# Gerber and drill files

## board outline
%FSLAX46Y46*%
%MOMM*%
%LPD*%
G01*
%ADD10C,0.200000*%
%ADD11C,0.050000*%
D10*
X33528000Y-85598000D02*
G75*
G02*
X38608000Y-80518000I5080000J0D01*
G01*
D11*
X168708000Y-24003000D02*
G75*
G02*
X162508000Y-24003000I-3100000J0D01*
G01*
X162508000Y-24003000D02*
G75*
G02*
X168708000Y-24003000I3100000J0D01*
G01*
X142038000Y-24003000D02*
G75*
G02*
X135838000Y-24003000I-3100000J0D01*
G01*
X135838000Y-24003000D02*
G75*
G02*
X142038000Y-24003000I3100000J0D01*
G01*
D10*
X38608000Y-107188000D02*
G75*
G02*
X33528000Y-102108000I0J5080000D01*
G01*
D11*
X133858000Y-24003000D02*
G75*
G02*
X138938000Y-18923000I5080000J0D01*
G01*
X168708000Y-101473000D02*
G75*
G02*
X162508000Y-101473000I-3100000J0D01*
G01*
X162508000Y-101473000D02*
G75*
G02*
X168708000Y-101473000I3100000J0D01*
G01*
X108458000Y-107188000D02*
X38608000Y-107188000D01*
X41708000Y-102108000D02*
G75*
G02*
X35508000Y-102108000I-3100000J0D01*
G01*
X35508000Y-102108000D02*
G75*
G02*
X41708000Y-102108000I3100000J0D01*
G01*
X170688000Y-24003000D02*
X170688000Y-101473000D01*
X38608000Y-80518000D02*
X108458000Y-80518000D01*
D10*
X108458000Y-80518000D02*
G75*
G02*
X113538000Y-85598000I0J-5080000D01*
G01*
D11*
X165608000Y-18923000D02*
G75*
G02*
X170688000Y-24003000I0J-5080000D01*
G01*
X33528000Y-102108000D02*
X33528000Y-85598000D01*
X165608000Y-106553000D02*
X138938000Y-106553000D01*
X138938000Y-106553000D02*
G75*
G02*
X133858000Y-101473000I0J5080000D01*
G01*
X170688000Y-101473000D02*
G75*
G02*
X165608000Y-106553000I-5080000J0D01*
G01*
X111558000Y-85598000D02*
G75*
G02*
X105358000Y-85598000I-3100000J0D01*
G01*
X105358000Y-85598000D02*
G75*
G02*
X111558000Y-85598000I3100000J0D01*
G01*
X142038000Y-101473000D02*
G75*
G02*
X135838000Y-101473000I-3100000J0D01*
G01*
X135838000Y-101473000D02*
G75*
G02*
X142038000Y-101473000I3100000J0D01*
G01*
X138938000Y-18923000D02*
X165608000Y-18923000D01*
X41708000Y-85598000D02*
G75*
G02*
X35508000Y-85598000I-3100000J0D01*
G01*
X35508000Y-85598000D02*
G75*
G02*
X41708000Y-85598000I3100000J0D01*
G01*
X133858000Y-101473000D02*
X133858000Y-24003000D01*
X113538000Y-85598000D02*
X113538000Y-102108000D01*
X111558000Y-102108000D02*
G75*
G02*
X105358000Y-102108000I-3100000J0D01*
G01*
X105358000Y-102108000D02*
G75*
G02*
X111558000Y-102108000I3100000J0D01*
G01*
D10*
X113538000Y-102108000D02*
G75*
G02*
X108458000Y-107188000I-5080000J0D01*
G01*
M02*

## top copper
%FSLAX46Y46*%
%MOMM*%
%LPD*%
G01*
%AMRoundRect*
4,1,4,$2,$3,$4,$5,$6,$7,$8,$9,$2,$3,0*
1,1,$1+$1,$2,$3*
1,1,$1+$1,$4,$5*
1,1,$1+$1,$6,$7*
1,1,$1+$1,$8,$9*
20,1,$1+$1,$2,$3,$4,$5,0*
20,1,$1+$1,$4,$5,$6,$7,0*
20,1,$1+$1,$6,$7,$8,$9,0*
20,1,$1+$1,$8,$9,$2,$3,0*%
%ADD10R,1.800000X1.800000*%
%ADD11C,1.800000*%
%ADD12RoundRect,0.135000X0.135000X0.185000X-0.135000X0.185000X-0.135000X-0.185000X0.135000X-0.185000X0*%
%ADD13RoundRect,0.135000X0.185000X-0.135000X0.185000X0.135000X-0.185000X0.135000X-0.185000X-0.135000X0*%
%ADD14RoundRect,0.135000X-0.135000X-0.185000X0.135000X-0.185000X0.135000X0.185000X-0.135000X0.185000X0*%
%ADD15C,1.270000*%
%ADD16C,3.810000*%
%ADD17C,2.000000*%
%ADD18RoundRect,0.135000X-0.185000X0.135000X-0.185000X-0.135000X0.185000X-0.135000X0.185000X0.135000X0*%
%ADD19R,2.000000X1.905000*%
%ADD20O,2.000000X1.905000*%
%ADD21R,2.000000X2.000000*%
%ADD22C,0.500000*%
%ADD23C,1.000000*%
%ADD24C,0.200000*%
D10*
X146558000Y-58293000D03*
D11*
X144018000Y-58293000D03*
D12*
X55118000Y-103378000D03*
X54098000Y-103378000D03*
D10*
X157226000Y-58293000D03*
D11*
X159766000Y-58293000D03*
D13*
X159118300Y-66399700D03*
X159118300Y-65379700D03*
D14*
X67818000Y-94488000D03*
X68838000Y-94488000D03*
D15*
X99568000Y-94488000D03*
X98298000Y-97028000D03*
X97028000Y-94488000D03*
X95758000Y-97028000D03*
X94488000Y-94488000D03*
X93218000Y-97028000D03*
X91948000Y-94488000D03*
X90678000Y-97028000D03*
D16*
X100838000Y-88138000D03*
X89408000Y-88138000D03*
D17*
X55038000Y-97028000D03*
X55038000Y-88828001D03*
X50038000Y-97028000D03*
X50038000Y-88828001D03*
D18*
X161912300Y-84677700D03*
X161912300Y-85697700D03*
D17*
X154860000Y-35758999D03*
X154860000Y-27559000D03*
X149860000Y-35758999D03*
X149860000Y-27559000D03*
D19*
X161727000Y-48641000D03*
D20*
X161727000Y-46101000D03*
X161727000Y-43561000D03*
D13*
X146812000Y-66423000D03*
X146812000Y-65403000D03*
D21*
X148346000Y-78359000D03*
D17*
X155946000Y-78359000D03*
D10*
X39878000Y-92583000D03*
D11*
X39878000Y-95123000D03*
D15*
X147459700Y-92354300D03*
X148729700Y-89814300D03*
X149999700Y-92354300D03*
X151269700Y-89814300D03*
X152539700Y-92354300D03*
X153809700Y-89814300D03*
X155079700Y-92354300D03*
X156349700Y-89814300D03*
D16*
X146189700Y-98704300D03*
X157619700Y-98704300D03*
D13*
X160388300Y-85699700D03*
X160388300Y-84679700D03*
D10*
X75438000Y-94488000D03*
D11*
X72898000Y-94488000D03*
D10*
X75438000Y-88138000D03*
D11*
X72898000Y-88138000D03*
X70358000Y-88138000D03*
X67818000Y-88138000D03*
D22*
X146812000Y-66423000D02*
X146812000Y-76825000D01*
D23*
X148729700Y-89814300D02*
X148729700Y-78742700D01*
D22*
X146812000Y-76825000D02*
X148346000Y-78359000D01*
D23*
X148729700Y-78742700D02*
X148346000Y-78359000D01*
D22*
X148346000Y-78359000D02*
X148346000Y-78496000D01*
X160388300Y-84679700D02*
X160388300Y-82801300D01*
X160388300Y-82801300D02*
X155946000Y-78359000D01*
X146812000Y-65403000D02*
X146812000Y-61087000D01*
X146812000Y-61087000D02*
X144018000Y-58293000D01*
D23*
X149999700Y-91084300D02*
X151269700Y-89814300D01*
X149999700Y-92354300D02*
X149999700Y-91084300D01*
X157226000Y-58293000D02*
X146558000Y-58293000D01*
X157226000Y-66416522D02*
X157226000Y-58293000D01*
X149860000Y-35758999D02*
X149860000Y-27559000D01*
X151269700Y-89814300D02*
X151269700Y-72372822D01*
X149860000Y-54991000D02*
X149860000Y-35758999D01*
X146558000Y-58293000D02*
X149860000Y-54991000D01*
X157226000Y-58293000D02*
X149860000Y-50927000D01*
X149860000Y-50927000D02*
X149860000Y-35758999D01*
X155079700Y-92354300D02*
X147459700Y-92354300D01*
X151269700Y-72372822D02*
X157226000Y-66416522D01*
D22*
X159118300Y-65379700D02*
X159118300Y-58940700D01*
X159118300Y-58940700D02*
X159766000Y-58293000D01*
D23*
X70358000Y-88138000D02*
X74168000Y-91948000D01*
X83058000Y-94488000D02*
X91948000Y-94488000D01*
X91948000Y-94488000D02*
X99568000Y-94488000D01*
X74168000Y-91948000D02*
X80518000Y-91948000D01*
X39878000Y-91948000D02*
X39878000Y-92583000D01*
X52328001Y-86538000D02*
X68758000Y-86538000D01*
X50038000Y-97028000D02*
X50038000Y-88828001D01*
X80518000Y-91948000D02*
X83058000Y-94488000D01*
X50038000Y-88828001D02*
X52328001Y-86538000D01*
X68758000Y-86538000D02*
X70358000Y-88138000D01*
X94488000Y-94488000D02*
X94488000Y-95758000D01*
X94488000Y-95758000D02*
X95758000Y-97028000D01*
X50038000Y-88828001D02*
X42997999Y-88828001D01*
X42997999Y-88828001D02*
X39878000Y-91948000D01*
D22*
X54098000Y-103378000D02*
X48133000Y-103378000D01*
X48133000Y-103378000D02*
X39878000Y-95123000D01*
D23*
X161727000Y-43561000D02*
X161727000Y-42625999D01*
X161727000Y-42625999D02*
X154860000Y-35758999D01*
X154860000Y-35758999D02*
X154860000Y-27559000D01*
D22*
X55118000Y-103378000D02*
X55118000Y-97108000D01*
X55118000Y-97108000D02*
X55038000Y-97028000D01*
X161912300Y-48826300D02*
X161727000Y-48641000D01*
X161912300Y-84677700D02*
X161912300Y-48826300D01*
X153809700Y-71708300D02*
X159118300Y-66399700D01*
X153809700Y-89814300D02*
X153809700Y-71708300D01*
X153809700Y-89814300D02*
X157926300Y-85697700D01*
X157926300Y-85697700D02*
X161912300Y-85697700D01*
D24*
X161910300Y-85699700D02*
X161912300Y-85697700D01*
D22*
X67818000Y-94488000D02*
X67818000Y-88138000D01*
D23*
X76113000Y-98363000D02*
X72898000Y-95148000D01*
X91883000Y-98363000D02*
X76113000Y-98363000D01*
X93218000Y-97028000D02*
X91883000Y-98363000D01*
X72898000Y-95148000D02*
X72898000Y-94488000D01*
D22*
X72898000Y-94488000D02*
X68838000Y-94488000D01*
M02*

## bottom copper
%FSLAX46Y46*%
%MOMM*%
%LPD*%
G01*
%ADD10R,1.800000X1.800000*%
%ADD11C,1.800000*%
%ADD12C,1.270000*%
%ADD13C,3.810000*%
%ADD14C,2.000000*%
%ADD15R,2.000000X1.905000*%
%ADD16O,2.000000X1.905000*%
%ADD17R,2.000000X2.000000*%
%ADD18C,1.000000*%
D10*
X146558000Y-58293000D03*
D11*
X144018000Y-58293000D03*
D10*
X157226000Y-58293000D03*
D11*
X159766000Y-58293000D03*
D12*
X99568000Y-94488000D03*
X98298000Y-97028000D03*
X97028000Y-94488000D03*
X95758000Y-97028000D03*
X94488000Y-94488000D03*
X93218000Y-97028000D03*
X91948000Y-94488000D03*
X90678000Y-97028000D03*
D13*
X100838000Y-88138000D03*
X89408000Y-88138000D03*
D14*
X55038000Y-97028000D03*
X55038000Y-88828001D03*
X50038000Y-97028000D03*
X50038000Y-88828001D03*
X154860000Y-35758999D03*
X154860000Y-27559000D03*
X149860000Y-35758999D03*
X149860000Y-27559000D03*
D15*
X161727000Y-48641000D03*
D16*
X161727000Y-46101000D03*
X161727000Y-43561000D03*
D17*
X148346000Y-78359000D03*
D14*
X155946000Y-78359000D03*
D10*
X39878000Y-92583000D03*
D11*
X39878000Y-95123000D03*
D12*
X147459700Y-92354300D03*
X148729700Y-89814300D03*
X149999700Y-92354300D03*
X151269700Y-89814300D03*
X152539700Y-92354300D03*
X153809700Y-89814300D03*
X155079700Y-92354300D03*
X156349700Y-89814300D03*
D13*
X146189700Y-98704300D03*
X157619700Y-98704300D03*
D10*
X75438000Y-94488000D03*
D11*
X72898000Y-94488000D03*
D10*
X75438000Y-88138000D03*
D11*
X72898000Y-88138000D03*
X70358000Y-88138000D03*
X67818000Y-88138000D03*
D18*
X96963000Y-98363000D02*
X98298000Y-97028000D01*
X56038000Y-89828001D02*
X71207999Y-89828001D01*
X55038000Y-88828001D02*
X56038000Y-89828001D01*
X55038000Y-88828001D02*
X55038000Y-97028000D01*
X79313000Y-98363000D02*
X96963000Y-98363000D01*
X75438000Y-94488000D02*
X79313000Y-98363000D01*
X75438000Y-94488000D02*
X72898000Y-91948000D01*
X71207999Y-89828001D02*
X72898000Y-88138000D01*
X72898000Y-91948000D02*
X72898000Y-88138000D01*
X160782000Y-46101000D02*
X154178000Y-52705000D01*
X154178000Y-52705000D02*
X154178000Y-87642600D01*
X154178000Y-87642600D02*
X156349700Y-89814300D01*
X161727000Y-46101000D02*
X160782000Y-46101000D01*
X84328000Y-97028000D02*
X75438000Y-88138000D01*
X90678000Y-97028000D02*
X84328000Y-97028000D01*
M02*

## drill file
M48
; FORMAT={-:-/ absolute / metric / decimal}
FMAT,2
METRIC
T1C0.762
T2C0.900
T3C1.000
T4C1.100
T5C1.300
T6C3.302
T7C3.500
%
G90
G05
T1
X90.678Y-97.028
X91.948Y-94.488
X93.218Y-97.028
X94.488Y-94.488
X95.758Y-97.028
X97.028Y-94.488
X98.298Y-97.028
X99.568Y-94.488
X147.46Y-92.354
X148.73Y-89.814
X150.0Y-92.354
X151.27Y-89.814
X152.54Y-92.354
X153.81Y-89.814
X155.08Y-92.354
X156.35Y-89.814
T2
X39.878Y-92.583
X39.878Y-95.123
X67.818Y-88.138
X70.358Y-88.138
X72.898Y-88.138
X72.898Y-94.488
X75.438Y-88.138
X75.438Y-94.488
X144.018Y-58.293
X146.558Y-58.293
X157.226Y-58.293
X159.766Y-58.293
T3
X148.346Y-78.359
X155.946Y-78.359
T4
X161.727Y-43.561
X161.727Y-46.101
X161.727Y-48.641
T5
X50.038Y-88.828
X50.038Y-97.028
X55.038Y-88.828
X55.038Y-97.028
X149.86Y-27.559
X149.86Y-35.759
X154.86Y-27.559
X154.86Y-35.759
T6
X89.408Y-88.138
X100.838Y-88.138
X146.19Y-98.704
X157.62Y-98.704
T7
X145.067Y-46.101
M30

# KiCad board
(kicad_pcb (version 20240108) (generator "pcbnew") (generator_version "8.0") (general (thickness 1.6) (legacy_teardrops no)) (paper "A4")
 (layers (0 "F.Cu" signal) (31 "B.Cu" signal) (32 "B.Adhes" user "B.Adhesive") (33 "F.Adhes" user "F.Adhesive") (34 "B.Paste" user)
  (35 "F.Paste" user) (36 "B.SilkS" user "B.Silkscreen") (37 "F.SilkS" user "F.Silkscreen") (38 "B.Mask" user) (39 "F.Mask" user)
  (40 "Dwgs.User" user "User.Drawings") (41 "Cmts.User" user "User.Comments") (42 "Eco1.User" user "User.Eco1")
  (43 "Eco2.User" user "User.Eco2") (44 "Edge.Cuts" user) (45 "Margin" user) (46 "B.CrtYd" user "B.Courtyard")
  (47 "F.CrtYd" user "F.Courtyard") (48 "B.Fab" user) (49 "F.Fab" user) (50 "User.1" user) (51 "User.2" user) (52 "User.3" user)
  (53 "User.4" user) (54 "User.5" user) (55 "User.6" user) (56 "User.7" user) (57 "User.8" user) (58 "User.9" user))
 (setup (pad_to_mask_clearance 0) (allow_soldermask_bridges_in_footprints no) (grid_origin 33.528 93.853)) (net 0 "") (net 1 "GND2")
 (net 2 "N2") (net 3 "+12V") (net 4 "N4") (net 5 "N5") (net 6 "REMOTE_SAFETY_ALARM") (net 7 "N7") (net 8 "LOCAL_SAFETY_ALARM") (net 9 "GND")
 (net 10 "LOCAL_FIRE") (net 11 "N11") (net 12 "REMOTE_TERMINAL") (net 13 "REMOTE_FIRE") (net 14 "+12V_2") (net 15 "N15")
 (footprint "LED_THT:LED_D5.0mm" (layer "F.Cu") (at 146.558 58.293 180)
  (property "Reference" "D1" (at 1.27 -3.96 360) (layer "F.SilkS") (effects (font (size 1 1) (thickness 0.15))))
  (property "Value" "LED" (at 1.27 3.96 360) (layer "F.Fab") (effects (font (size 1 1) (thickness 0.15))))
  (pad "1" thru_hole rect (at 0 0 180) (size 1.8 1.8) (drill 0.9) (layers "*.Cu" "*.Mask") (remove_unused_layers no) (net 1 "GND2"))
  (pad "2" thru_hole circle (at 2.54 0 180) (size 1.8 1.8) (drill 0.9) (layers "*.Cu" "*.Mask") (remove_unused_layers no) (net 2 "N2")))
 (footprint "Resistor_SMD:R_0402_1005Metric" (layer "F.Cu") (at 54.608 103.378 180)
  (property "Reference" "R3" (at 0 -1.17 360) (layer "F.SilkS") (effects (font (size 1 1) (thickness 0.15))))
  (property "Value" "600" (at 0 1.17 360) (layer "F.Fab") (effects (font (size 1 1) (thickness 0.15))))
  (pad "1" smd roundrect (at -0.51 0 180) (size 0.54 0.64) (layers "F.Cu" "F.Paste" "F.Mask") (roundrect_rratio 0.25) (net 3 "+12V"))
  (pad "2" smd roundrect (at 0.51 0 180) (size 0.54 0.64) (layers "F.Cu" "F.Paste" "F.Mask") (roundrect_rratio 0.25) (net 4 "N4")))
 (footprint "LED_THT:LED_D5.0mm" (layer "F.Cu") (at 157.226 58.293)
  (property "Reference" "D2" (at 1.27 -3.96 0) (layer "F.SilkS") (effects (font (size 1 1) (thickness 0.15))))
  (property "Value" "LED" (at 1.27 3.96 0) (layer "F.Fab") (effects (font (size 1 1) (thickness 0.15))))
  (pad "1" thru_hole rect (at 0 0) (size 1.8 1.8) (drill 0.9) (layers "*.Cu" "*.Mask") (remove_unused_layers no) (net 1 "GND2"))
  (pad "2" thru_hole circle (at 2.54 0) (size 1.8 1.8) (drill 0.9) (layers "*.Cu" "*.Mask") (remove_unused_layers no) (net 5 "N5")))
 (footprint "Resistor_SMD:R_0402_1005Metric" (layer "F.Cu") (at 159.1183 65.8897 90)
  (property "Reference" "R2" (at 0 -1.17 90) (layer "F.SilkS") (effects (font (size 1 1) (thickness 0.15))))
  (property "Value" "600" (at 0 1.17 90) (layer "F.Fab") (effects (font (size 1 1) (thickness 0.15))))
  (pad "1" smd roundrect (at -0.51 0 90) (size 0.54 0.64) (layers "F.Cu" "F.Paste" "F.Mask") (roundrect_rratio 0.25)
   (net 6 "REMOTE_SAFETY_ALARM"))
  (pad "2" smd roundrect (at 0.51 0 90) (size 0.54 0.64) (layers "F.Cu" "F.Paste" "F.Mask") (roundrect_rratio 0.25) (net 5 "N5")))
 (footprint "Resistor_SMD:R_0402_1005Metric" (layer "F.Cu") (at 68.328 94.488)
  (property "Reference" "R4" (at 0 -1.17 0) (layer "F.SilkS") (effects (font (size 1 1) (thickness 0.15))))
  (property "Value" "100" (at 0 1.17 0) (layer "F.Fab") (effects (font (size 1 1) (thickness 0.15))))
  (pad "1" smd roundrect (at -0.51 0) (size 0.54 0.64) (layers "F.Cu" "F.Paste" "F.Mask") (roundrect_rratio 0.25) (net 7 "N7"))
  (pad "2" smd roundrect (at 0.51 0) (size 0.54 0.64) (layers "F.Cu" "F.Paste" "F.Mask") (roundrect_rratio 0.25)
   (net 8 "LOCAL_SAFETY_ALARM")))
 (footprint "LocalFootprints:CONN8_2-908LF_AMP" (layer "F.Cu") (at 99.568 94.488 180)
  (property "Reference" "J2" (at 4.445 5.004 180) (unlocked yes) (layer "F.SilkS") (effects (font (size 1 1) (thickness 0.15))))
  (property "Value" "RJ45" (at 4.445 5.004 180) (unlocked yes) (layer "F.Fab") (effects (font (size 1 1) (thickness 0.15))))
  (pad "1" thru_hole circle (at 0 0 180) (size 1.27 1.27) (drill 0.762) (layers "*.Cu" "*.Mask") (remove_unused_layers no) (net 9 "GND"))
  (pad "2" thru_hole circle (at 1.27 -2.54 180) (size 1.27 1.27) (drill 0.762) (layers "*.Cu" "*.Mask") (remove_unused_layers no)
   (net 3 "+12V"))
  (pad "3" thru_hole circle (at 2.54 0 180) (size 1.27 1.27) (drill 0.762) (layers "*.Cu" "*.Mask") (remove_unused_layers no) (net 9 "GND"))
  (pad "4" thru_hole circle (at 3.81 -2.54 180) (size 1.27 1.27) (drill 0.762) (layers "*.Cu" "*.Mask") (remove_unused_layers no)
   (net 9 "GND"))
  (pad "5" thru_hole circle (at 5.08 0 180) (size 1.27 1.27) (drill 0.762) (layers "*.Cu" "*.Mask") (remove_unused_layers no) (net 9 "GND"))
  (pad "6" thru_hole circle (at 6.35 -2.54 180) (size 1.27 1.27) (drill 0.762) (layers "*.Cu" "*.Mask") (remove_unused_layers no)
   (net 8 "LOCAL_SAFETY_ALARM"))
  (pad "7" thru_hole circle (at 7.62 0 180) (size 1.27 1.27) (drill 0.762) (layers "*.Cu" "*.Mask") (remove_unused_layers no) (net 9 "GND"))
  (pad "8" thru_hole circle (at 8.89 -2.54 180) (size 1.27 1.27) (drill 0.762) (layers "*.Cu" "*.Mask") (remove_unused_layers no)
   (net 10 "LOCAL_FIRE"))
  (pad "9" thru_hole circle (at -1.27 6.35 270) (size 3.81 3.81) (drill 3.302) (layers "*.Cu" "*.Mask") (remove_unused_layers no))
  (pad "10" thru_hole circle (at 10.16 6.35 270) (size 3.81 3.81) (drill 3.302) (layers "*.Cu" "*.Mask") (remove_unused_layers no)))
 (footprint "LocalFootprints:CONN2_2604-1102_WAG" (layer "F.Cu") (at 55.038 97.028 180)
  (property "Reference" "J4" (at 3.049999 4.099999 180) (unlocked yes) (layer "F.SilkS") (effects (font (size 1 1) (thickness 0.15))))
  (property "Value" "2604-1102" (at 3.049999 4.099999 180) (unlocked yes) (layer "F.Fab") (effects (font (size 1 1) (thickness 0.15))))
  (pad "1" thru_hole circle (at 0 0 180) (size 2 2) (drill 1.3) (layers "*.Cu" "*.Mask") (remove_unused_layers no) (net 3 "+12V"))
  (pad "2" thru_hole circle (at 0 8.199999 180) (size 2 2) (drill 1.3) (layers "*.Cu" "*.Mask") (remove_unused_layers no) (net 3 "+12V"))
  (pad "3" thru_hole circle (at 5 0 180) (size 2 2) (drill 1.3) (layers "*.Cu" "*.Mask") (remove_unused_layers no) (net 9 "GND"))
  (pad "4" thru_hole circle (at 5 8.199999 180) (size 2 2) (drill 1.3) (layers "*.Cu" "*.Mask") (remove_unused_layers no) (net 9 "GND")))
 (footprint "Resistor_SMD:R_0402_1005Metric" (layer "F.Cu") (at 161.9123 85.1877 -90)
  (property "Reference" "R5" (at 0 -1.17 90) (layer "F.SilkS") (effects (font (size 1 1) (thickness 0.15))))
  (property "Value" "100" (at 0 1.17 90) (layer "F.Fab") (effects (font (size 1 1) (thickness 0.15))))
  (pad "1" smd roundrect (at -0.51 0 270) (size 0.54 0.64) (layers "F.Cu" "F.Paste" "F.Mask") (roundrect_rratio 0.25) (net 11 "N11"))
  (pad "2" smd roundrect (at 0.51 0 270) (size 0.54 0.64) (layers "F.Cu" "F.Paste" "F.Mask") (roundrect_rratio 0.25)
   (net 6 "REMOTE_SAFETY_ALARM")))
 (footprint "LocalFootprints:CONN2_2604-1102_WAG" (layer "F.Cu") (at 154.86 35.758999 180)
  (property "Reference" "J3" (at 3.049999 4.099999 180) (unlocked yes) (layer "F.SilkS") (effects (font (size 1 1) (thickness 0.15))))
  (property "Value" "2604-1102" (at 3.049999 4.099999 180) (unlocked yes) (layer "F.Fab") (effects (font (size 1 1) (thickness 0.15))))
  (pad "1" thru_hole circle (at 0 0 180) (size 2 2) (drill 1.3) (layers "*.Cu" "*.Mask") (remove_unused_layers no)
   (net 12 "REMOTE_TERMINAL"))
  (pad "2" thru_hole circle (at 0 8.199999 180) (size 2 2) (drill 1.3) (layers "*.Cu" "*.Mask") (remove_unused_layers no)
   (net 12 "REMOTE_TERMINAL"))
  (pad "3" thru_hole circle (at 5 0 180) (size 2 2) (drill 1.3) (layers "*.Cu" "*.Mask") (remove_unused_layers no) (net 1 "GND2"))
  (pad "4" thru_hole circle (at 5 8.199999 180) (size 2 2) (drill 1.3) (layers "*.Cu" "*.Mask") (remove_unused_layers no) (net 1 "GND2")))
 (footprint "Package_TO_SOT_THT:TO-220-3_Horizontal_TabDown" (layer "F.Cu") (at 161.727 48.641 90)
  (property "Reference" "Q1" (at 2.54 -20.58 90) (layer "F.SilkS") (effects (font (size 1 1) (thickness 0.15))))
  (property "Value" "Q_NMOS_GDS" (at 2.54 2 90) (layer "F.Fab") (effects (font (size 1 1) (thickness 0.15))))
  (pad "" np_thru_hole oval (at 2.54 -16.66 90) (size 3.5 3.5) (drill 3.5) (layers "*.Cu" "*.Mask"))
  (pad "1" thru_hole rect (at 0 0 90) (size 1.905 2) (drill 1.1) (layers "*.Cu" "*.Mask") (remove_unused_layers no) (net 11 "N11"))
  (pad "2" thru_hole oval (at 2.54 0 90) (size 1.905 2) (drill 1.1) (layers "*.Cu" "*.Mask") (remove_unused_layers no)
   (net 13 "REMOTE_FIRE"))
  (pad "3" thru_hole oval (at 5.08 0 90) (size 1.905 2) (drill 1.1) (layers "*.Cu" "*.Mask") (remove_unused_layers no)
   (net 12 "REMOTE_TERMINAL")))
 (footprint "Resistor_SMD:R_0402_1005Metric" (layer "F.Cu") (at 146.812 65.913 90)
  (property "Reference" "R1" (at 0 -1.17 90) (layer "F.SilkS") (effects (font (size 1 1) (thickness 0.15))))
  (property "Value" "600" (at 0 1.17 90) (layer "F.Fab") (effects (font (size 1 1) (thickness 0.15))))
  (pad "1" smd roundrect (at -0.51 0 90) (size 0.54 0.64) (layers "F.Cu" "F.Paste" "F.Mask") (roundrect_rratio 0.25) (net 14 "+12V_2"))
  (pad "2" smd roundrect (at 0.51 0 90) (size 0.54 0.64) (layers "F.Cu" "F.Paste" "F.Mask") (roundrect_rratio 0.25) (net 2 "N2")))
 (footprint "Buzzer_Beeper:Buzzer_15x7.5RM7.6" (layer "F.Cu") (at 148.346 78.359)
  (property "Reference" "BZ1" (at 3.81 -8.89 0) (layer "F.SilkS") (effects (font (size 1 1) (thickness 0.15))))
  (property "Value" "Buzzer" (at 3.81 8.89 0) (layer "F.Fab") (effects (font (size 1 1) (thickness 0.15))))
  (pad "1" thru_hole rect (at 0 0) (size 2 2) (drill 1) (layers "*.Cu" "*.Mask") (remove_unused_layers no) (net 14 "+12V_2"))
  (pad "2" thru_hole circle (at 7.6 0) (size 2 2) (drill 1) (layers "*.Cu" "*.Mask") (remove_unused_layers no) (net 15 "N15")))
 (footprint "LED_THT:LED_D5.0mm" (layer "F.Cu") (at 39.878 92.583 -90)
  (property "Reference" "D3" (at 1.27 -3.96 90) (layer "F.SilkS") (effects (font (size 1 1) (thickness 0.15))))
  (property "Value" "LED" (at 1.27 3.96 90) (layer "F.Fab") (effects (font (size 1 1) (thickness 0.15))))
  (pad "1" thru_hole rect (at 0 0 270) (size 1.8 1.8) (drill 0.9) (layers "*.Cu" "*.Mask") (remove_unused_layers no) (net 9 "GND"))
  (pad "2" thru_hole circle (at 2.54 0 270) (size 1.8 1.8) (drill 0.9) (layers "*.Cu" "*.Mask") (remove_unused_layers no) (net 4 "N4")))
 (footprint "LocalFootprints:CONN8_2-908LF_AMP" (layer "F.Cu") (at 147.4597 92.3543)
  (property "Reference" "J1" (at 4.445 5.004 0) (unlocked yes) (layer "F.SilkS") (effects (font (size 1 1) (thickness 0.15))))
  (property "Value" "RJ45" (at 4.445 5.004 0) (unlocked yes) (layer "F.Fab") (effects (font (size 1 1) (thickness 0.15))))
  (pad "1" thru_hole circle (at 0 0) (size 1.27 1.27) (drill 0.762) (layers "*.Cu" "*.Mask") (remove_unused_layers no) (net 1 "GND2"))
  (pad "2" thru_hole circle (at 1.27 -2.54) (size 1.27 1.27) (drill 0.762) (layers "*.Cu" "*.Mask") (remove_unused_layers no)
   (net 14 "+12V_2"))
  (pad "3" thru_hole circle (at 2.54 0) (size 1.27 1.27) (drill 0.762) (layers "*.Cu" "*.Mask") (remove_unused_layers no) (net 1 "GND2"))
  (pad "4" thru_hole circle (at 3.81 -2.54) (size 1.27 1.27) (drill 0.762) (layers "*.Cu" "*.Mask") (remove_unused_layers no) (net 1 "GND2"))
  (pad "5" thru_hole circle (at 5.08 0) (size 1.27 1.27) (drill 0.762) (layers "*.Cu" "*.Mask") (remove_unused_layers no) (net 1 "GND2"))
  (pad "6" thru_hole circle (at 6.35 -2.54) (size 1.27 1.27) (drill 0.762) (layers "*.Cu" "*.Mask") (remove_unused_layers no)
   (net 6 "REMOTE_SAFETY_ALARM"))
  (pad "7" thru_hole circle (at 7.62 0) (size 1.27 1.27) (drill 0.762) (layers "*.Cu" "*.Mask") (remove_unused_layers no) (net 1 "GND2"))
  (pad "8" thru_hole circle (at 8.89 -2.54) (size 1.27 1.27) (drill 0.762) (layers "*.Cu" "*.Mask") (remove_unused_layers no)
   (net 13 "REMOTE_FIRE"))
  (pad "9" thru_hole circle (at -1.27 6.35 90) (size 3.81 3.81) (drill 3.302) (layers "*.Cu" "*.Mask") (remove_unused_layers no))
  (pad "10" thru_hole circle (at 10.16 6.35 90) (size 3.81 3.81) (drill 3.302) (layers "*.Cu" "*.Mask") (remove_unused_layers no)))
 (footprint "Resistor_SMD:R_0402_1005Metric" (layer "F.Cu") (at 160.3883 85.1897 90)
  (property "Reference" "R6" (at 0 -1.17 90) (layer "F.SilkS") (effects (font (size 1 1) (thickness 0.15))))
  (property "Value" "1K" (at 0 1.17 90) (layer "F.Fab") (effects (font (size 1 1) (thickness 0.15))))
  (pad "1" smd roundrect (at -0.51 0 90) (size 0.54 0.64) (layers "F.Cu" "F.Paste" "F.Mask") (roundrect_rratio 0.25)
   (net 6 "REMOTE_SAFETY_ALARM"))
  (pad "2" smd roundrect (at 0.51 0 90) (size 0.54 0.64) (layers "F.Cu" "F.Paste" "F.Mask") (roundrect_rratio 0.25) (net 15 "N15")))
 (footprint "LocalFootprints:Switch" (layer "B.Cu") (at 75.438 94.488 180)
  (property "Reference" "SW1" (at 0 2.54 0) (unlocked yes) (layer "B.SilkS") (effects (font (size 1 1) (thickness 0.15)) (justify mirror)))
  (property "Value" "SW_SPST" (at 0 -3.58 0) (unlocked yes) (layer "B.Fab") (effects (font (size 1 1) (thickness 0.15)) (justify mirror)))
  (pad "1" thru_hole rect (at 0 0 180) (size 1.8 1.8) (drill 0.9) (layers "*.Cu" "*.Mask") (remove_unused_layers no) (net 3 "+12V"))
  (pad "2" thru_hole circle (at 2.54 0 180) (size 1.8 1.8) (drill 0.9) (layers "*.Cu" "*.Mask") (remove_unused_layers no)
   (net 8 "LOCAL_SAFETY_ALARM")))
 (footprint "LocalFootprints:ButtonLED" (layer "B.Cu") (at 75.438 88.138 180)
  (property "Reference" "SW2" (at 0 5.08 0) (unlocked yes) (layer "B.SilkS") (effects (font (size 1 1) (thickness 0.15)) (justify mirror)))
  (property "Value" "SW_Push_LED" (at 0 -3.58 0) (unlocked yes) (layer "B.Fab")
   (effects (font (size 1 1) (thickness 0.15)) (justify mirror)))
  (pad "1" thru_hole rect (at 0 0 180) (size 1.8 1.8) (drill 0.9) (layers "*.Cu" "*.Mask") (remove_unused_layers no) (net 10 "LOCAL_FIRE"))
  (pad "2" thru_hole circle (at 2.54 0 180) (size 1.8 1.8) (drill 0.9) (layers "*.Cu" "*.Mask") (remove_unused_layers no) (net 3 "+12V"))
  (pad "3" thru_hole circle (at 5.08 0 180) (size 1.8 1.8) (drill 0.9) (layers "*.Cu" "*.Mask") (remove_unused_layers no) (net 9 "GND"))
  (pad "4" thru_hole circle (at 7.62 0 180) (size 1.8 1.8) (drill 0.9) (layers "*.Cu" "*.Mask") (remove_unused_layers no) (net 7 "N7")))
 (gr_arc (start 33.528 85.598) (mid 35.015898 82.005898) (end 38.608 80.518) (stroke (width 0.2) (type default)) (layer "Edge.Cuts"))
 (gr_circle (center 165.608 24.003) (end 168.708 24.003) (stroke (width 0.05) (type default)) (fill none) (layer "Edge.Cuts"))
 (gr_circle (center 138.938 24.003) (end 142.038 24.003) (stroke (width 0.05) (type default)) (fill none) (layer "Edge.Cuts"))
 (gr_arc (start 38.608 107.188) (mid 35.015898 105.700102) (end 33.528 102.108) (stroke (width 0.2) (type default)) (layer "Edge.Cuts"))
 (gr_arc (start 133.858 24.003) (mid 135.345898 20.410898) (end 138.938 18.923) (stroke (width 0.05) (type default)) (layer "Edge.Cuts"))
 (gr_circle (center 165.608 101.473) (end 168.708 101.473) (stroke (width 0.05) (type default)) (fill none) (layer "Edge.Cuts"))
 (gr_line (start 108.458 107.188) (end 38.608 107.188) (stroke (width 0.05) (type default)) (layer "Edge.Cuts"))
 (gr_circle (center 38.608 102.108) (end 41.708 102.108) (stroke (width 0.05) (type default)) (fill none) (layer "Edge.Cuts"))
 (gr_line (start 170.688 24.003) (end 170.688 101.473) (stroke (width 0.05) (type default)) (layer "Edge.Cuts"))
 (gr_line (start 38.608 80.518) (end 108.458 80.518) (stroke (width 0.05) (type default)) (layer "Edge.Cuts"))
 (gr_arc (start 108.458 80.518) (mid 112.050102 82.005898) (end 113.538 85.598) (stroke (width 0.2) (type default)) (layer "Edge.Cuts"))
 (gr_arc (start 165.608 18.923) (mid 169.200102 20.410898) (end 170.688 24.003) (stroke (width 0.05) (type default)) (layer "Edge.Cuts"))
 (gr_line (start 33.528 102.108) (end 33.528 85.598) (stroke (width 0.05) (type default)) (layer "Edge.Cuts"))
 (gr_line (start 165.608 106.553) (end 138.938 106.553) (stroke (width 0.05) (type default)) (layer "Edge.Cuts"))
 (gr_arc (start 138.938 106.553) (mid 135.345898 105.065102) (end 133.858 101.473) (stroke (width 0.05) (type default)) (layer "Edge.Cuts"))
 (gr_arc (start 170.688 101.473) (mid 169.200102 105.065102) (end 165.608 106.553) (stroke (width 0.05) (type default)) (layer "Edge.Cuts"))
 (gr_circle (center 108.458 85.598) (end 111.558 85.598) (stroke (width 0.05) (type default)) (fill none) (layer "Edge.Cuts"))
 (gr_circle (center 138.938 101.473) (end 142.038 101.473) (stroke (width 0.05) (type default)) (fill none) (layer "Edge.Cuts"))
 (gr_line (start 138.938 18.923) (end 165.608 18.923) (stroke (width 0.05) (type default)) (layer "Edge.Cuts"))
 (gr_circle (center 38.608 85.598) (end 41.708 85.598) (stroke (width 0.05) (type default)) (fill none) (layer "Edge.Cuts"))
 (gr_line (start 133.858 101.473) (end 133.858 24.003) (stroke (width 0.05) (type default)) (layer "Edge.Cuts"))
 (gr_line (start 113.538 85.598) (end 113.538 102.108) (stroke (width 0.05) (type default)) (layer "Edge.Cuts"))
 (gr_circle (center 108.458 102.108) (end 111.558 102.108) (stroke (width 0.05) (type default)) (fill none) (layer "Edge.Cuts"))
 (gr_arc (start 113.538 102.108) (mid 112.050102 105.700102) (end 108.458 107.188) (stroke (width 0.2) (type default)) (layer "Edge.Cuts"))
 (segment (start 146.812 66.423) (end 146.812 76.825) (width 0.5) (layer "F.Cu") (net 14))
 (segment (start 148.7297 89.8143) (end 148.7297 78.7427) (width 1) (layer "F.Cu") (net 14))
 (segment (start 146.812 76.825) (end 148.346 78.359) (width 0.5) (layer "F.Cu") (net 14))
 (segment (start 148.7297 78.7427) (end 148.346 78.359) (width 1) (layer "F.Cu") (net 14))
 (segment (start 148.346 78.359) (end 148.346 78.496) (width 0.5) (layer "F.Cu") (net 14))
 (segment (start 160.3883 84.6797) (end 160.3883 82.8013) (width 0.5) (layer "F.Cu") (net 15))
 (segment (start 160.3883 82.8013) (end 155.946 78.359) (width 0.5) (layer "F.Cu") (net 15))
 (segment (start 146.812 65.403) (end 146.812 61.087) (width 0.5) (layer "F.Cu") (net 2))
 (segment (start 146.812 61.087) (end 144.018 58.293) (width 0.5) (layer "F.Cu") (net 2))
 (segment (start 149.9997 91.0843) (end 151.2697 89.8143) (width 1) (layer "F.Cu") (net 1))
 (segment (start 149.9997 92.3543) (end 149.9997 91.0843) (width 1) (layer "F.Cu") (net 1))
 (segment (start 157.226 58.293) (end 146.558 58.293) (width 1) (layer "F.Cu") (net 1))
 (segment (start 157.226 66.416522) (end 157.226 58.293) (width 1) (layer "F.Cu") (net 1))
 (segment (start 149.86 35.758999) (end 149.86 27.559) (width 1) (layer "F.Cu") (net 1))
 (segment (start 151.2697 89.8143) (end 151.2697 72.372822) (width 1) (layer "F.Cu") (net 1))
 (segment (start 149.86 54.991) (end 149.86 35.758999) (width 1) (layer "F.Cu") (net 1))
 (segment (start 146.558 58.293) (end 149.86 54.991) (width 1) (layer "F.Cu") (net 1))
 (segment (start 157.226 58.293) (end 149.86 50.927) (width 1) (layer "F.Cu") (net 1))
 (segment (start 149.86 50.927) (end 149.86 35.758999) (width 1) (layer "F.Cu") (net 1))
 (segment (start 155.0797 92.3543) (end 147.4597 92.3543) (width 1) (layer "F.Cu") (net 1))
 (segment (start 151.2697 72.372822) (end 157.226 66.416522) (width 1) (layer "F.Cu") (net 1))
 (segment (start 159.1183 65.3797) (end 159.1183 58.9407) (width 0.5) (layer "F.Cu") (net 5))
 (segment (start 159.1183 58.9407) (end 159.766 58.293) (width 0.5) (layer "F.Cu") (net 5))
 (segment (start 70.358 88.138) (end 74.168 91.948) (width 1) (layer "F.Cu") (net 9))
 (segment (start 83.058 94.488) (end 91.948 94.488) (width 1) (layer "F.Cu") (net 9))
 (segment (start 91.948 94.488) (end 99.568 94.488) (width 1) (layer "F.Cu") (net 9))
 (segment (start 74.168 91.948) (end 80.518 91.948) (width 1) (layer "F.Cu") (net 9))
 (segment (start 39.878 91.948) (end 39.878 92.583) (width 1) (layer "F.Cu") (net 9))
 (segment (start 52.328001 86.538) (end 68.758 86.538) (width 1) (layer "F.Cu") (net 9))
 (segment (start 50.038 97.028) (end 50.038 88.828001) (width 1) (layer "F.Cu") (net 9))
 (segment (start 80.518 91.948) (end 83.058 94.488) (width 1) (layer "F.Cu") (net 9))
 (segment (start 50.038 88.828001) (end 52.328001 86.538) (width 1) (layer "F.Cu") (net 9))
 (segment (start 68.758 86.538) (end 70.358 88.138) (width 1) (layer "F.Cu") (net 9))
 (segment (start 94.488 94.488) (end 94.488 95.758) (width 1) (layer "F.Cu") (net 9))
 (segment (start 94.488 95.758) (end 95.758 97.028) (width 1) (layer "F.Cu") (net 9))
 (segment (start 50.038 88.828001) (end 42.997999 88.828001) (width 1) (layer "F.Cu") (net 9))
 (segment (start 42.997999 88.828001) (end 39.878 91.948) (width 1) (layer "F.Cu") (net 9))
 (segment (start 54.098 103.378) (end 48.133 103.378) (width 0.5) (layer "F.Cu") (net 4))
 (segment (start 48.133 103.378) (end 39.878 95.123) (width 0.5) (layer "F.Cu") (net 4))
 (segment (start 161.727 43.561) (end 161.727 42.625999) (width 1) (layer "F.Cu") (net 12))
 (segment (start 161.727 42.625999) (end 154.86 35.758999) (width 1) (layer "F.Cu") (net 12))
 (segment (start 154.86 35.758999) (end 154.86 27.559) (width 1) (layer "F.Cu") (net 12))
 (segment (start 55.118 103.378) (end 55.118 97.108) (width 0.5) (layer "F.Cu") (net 3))
 (segment (start 55.118 97.108) (end 55.038 97.028) (width 0.5) (layer "F.Cu") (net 3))
 (segment (start 96.963 98.363) (end 98.298 97.028) (width 1) (layer "B.Cu") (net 3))
 (segment (start 56.038 89.828001) (end 71.207999 89.828001) (width 1) (layer "B.Cu") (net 3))
 (segment (start 55.038 88.828001) (end 56.038 89.828001) (width 1) (layer "B.Cu") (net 3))
 (segment (start 55.038 88.828001) (end 55.038 97.028) (width 1) (layer "B.Cu") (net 3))
 (segment (start 79.313 98.363) (end 96.963 98.363) (width 1) (layer "B.Cu") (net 3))
 (segment (start 75.438 94.488) (end 79.313 98.363) (width 1) (layer "B.Cu") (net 3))
 (segment (start 75.438 94.488) (end 72.898 91.948) (width 1) (layer "B.Cu") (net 3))
 (segment (start 71.207999 89.828001) (end 72.898 88.138) (width 1) (layer "B.Cu") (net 3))
 (segment (start 72.898 91.948) (end 72.898 88.138) (width 1) (layer "B.Cu") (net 3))
 (segment (start 160.782 46.101) (end 154.178 52.705) (width 1) (layer "B.Cu") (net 13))
 (segment (start 154.178 52.705) (end 154.178 87.6426) (width 1) (layer "B.Cu") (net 13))
 (segment (start 154.178 87.6426) (end 156.3497 89.8143) (width 1) (layer "B.Cu") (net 13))
 (segment (start 161.727 46.101) (end 160.782 46.101) (width 1) (layer "B.Cu") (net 13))
 (segment (start 161.9123 48.8263) (end 161.727 48.641) (width 0.5) (layer "F.Cu") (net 11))
 (segment (start 161.9123 84.6777) (end 161.9123 48.8263) (width 0.5) (layer "F.Cu") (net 11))
 (segment (start 153.8097 71.7083) (end 159.1183 66.3997) (width 0.5) (layer "F.Cu") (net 6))
 (segment (start 153.8097 89.8143) (end 153.8097 71.7083) (width 0.5) (layer "F.Cu") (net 6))
 (segment (start 153.8097 89.8143) (end 157.9263 85.6977) (width 0.5) (layer "F.Cu") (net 6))
 (segment (start 157.9263 85.6977) (end 161.9123 85.6977) (width 0.5) (layer "F.Cu") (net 6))
 (segment (start 161.9103 85.6997) (end 161.9123 85.6977) (width 0.2) (layer "F.Cu") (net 6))
 (segment (start 67.818 94.488) (end 67.818 88.138) (width 0.5) (layer "F.Cu") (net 7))
 (segment (start 76.113 98.363) (end 72.898 95.148) (width 1) (layer "F.Cu") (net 8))
 (segment (start 91.883 98.363) (end 76.113 98.363) (width 1) (layer "F.Cu") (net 8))
 (segment (start 93.218 97.028) (end 91.883 98.363) (width 1) (layer "F.Cu") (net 8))
 (segment (start 72.898 95.148) (end 72.898 94.488) (width 1) (layer "F.Cu") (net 8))
 (segment (start 72.898 94.488) (end 68.838 94.488) (width 0.5) (layer "F.Cu") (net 8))
 (segment (start 84.328 97.028) (end 75.438 88.138) (width 1) (layer "B.Cu") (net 10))
 (segment (start 90.678 97.028) (end 84.328 97.028) (width 1) (layer "B.Cu") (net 10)))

